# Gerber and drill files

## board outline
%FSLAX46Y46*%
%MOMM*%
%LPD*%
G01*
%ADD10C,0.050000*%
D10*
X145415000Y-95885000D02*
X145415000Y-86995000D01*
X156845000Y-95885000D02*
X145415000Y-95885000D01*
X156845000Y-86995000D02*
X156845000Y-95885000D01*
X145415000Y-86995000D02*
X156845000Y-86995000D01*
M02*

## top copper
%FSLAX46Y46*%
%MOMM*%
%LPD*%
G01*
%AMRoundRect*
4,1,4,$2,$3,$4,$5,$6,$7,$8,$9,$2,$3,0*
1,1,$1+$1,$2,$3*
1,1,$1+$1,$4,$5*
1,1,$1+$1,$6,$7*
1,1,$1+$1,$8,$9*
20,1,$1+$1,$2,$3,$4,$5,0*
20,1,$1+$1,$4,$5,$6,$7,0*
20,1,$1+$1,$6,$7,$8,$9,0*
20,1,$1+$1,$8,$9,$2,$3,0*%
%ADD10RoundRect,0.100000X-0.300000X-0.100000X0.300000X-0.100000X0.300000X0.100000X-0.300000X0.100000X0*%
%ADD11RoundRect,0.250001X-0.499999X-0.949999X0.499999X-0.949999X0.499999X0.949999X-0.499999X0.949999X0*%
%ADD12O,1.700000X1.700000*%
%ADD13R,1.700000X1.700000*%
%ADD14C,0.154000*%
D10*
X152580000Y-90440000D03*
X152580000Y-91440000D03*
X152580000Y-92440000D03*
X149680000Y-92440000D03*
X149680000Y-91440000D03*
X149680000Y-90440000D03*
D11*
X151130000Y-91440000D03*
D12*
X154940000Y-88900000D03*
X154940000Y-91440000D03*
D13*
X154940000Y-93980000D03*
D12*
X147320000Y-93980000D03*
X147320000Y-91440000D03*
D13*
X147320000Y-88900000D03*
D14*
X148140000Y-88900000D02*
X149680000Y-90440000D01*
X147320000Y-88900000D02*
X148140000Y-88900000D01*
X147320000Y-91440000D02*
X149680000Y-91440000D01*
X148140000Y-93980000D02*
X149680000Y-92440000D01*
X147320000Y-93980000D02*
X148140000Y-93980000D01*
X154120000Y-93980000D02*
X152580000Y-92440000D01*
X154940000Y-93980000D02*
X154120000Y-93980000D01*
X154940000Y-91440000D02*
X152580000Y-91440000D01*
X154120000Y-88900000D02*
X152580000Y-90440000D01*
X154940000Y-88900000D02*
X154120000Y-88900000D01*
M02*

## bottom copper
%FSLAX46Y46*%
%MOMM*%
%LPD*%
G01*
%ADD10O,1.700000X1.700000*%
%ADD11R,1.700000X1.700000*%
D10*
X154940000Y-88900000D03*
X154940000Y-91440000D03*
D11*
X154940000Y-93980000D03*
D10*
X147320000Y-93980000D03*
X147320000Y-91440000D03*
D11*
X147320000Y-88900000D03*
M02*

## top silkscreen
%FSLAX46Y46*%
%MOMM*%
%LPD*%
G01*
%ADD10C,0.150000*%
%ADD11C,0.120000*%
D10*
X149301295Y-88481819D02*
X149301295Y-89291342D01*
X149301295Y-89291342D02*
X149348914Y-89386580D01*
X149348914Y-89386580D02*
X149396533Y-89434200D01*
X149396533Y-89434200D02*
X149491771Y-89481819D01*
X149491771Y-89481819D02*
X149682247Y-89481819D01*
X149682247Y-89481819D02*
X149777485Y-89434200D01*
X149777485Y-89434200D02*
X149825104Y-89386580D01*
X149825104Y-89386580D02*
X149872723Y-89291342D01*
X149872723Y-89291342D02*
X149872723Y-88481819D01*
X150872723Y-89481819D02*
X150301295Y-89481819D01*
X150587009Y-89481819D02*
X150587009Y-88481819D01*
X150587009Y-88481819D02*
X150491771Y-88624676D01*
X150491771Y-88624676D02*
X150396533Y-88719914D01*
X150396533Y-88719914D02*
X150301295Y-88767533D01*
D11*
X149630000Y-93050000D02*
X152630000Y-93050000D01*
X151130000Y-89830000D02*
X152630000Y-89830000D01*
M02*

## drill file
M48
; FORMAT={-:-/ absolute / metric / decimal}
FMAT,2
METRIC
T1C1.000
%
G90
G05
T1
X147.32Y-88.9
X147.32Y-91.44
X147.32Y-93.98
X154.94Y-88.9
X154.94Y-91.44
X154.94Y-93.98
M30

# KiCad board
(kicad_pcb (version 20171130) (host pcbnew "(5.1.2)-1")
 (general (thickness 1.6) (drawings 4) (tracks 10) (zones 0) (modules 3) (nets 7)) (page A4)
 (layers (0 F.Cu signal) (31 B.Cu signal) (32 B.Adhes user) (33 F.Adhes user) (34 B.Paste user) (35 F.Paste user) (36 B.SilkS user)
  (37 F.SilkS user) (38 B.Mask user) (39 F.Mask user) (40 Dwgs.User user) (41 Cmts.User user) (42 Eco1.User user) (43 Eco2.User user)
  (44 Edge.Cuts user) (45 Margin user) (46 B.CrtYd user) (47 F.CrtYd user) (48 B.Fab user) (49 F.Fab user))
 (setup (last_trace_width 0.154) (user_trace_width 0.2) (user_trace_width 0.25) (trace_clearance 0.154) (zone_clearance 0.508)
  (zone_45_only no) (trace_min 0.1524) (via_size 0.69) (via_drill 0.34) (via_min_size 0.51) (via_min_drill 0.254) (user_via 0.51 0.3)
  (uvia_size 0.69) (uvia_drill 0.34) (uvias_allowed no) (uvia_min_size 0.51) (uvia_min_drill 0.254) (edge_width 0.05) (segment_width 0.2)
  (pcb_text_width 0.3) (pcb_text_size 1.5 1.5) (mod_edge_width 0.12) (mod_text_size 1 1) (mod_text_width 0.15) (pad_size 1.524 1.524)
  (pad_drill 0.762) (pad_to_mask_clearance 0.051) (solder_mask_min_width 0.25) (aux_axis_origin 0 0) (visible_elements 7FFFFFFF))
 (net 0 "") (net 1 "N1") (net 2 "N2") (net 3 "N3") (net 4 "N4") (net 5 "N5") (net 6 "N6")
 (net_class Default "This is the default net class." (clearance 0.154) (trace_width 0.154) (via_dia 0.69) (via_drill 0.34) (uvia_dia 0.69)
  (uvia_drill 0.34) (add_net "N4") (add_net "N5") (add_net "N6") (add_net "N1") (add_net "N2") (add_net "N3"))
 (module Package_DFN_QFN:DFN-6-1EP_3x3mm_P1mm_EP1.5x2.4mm (layer F.Cu) (at 151.13 91.44)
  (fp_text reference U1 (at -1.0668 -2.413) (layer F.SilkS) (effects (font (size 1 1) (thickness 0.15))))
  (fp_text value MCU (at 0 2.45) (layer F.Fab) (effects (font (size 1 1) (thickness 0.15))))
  (fp_line (start -1.5 1.61) (end 1.5 1.61) (layer F.SilkS) (width 0.12))
  (fp_line (start 0 -1.61) (end 1.5 -1.61) (layer F.SilkS) (width 0.12))
  (pad 6 smd roundrect (at 1.45 -1) (size 0.8 0.4) (layers F.Cu F.Paste F.Mask) (roundrect_rratio 0.25) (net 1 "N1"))
  (pad 5 smd roundrect (at 1.45 0) (size 0.8 0.4) (layers F.Cu F.Paste F.Mask) (roundrect_rratio 0.25) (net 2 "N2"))
  (pad 4 smd roundrect (at 1.45 1) (size 0.8 0.4) (layers F.Cu F.Paste F.Mask) (roundrect_rratio 0.25) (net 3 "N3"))
  (pad 3 smd roundrect (at -1.45 1) (size 0.8 0.4) (layers F.Cu F.Paste F.Mask) (roundrect_rratio 0.25) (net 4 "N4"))
  (pad 2 smd roundrect (at -1.45 0) (size 0.8 0.4) (layers F.Cu F.Paste F.Mask) (roundrect_rratio 0.25) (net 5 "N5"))
  (pad 1 smd roundrect (at -1.45 -1) (size 0.8 0.4) (layers F.Cu F.Paste F.Mask) (roundrect_rratio 0.25) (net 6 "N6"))
  (pad "" smd roundrect (at 0.375 0.6) (size 0.6 0.97) (layers F.Paste) (roundrect_rratio 0.25))
  (pad "" smd roundrect (at 0.375 -0.6) (size 0.6 0.97) (layers F.Paste) (roundrect_rratio 0.25))
  (pad "" smd roundrect (at -0.375 0.6) (size 0.6 0.97) (layers F.Paste) (roundrect_rratio 0.25))
  (pad "" smd roundrect (at -0.375 -0.6) (size 0.6 0.97) (layers F.Paste) (roundrect_rratio 0.25))
  (pad 7 smd roundrect (at 0 0) (size 1.5 2.4) (layers F.Cu F.Mask) (roundrect_rratio 0.166667)))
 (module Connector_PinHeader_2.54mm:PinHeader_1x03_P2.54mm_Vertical (layer B.Cu) (at 154.94 93.98)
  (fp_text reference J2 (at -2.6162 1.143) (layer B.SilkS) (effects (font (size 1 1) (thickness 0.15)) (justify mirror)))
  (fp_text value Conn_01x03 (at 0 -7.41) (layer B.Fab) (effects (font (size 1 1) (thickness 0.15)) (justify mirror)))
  (pad 3 thru_hole oval (at 0 -5.08) (size 1.7 1.7) (drill 1) (layers *.Cu *.Mask) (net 3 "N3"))
  (pad 2 thru_hole oval (at 0 -2.54) (size 1.7 1.7) (drill 1) (layers *.Cu *.Mask) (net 2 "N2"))
  (pad 1 thru_hole rect (at 0 0) (size 1.7 1.7) (drill 1) (layers *.Cu *.Mask) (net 1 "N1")))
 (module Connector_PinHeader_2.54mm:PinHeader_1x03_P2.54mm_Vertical (layer B.Cu) (at 147.32 88.9 180)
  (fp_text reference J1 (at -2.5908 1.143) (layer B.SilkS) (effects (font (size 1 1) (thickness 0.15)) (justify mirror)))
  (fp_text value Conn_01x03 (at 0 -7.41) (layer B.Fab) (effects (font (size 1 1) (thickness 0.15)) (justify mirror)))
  (pad 3 thru_hole oval (at 0 -5.08 180) (size 1.7 1.7) (drill 1) (layers *.Cu *.Mask) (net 6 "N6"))
  (pad 2 thru_hole oval (at 0 -2.54 180) (size 1.7 1.7) (drill 1) (layers *.Cu *.Mask) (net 5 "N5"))
  (pad 1 thru_hole rect (at 0 0 180) (size 1.7 1.7) (drill 1) (layers *.Cu *.Mask) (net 4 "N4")))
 (gr_line (start 145.415 95.885) (end 145.415 86.995) (layer Edge.Cuts) (width 0.05))
 (gr_line (start 156.845 95.885) (end 145.415 95.885) (layer Edge.Cuts) (width 0.05))
 (gr_line (start 156.845 86.995) (end 156.845 95.885) (layer Edge.Cuts) (width 0.05))
 (gr_line (start 145.415 86.995) (end 156.845 86.995) (layer Edge.Cuts) (width 0.05))
 (segment (start 148.14 88.9) (end 149.68 90.44) (width 0.154) (layer F.Cu) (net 6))
 (segment (start 147.32 88.9) (end 148.14 88.9) (width 0.154) (layer F.Cu) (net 6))
 (segment (start 147.32 91.44) (end 149.68 91.44) (width 0.154) (layer F.Cu) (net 5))
 (segment (start 148.14 93.98) (end 149.68 92.44) (width 0.154) (layer F.Cu) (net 4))
 (segment (start 147.32 93.98) (end 148.14 93.98) (width 0.154) (layer F.Cu) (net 4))
 (segment (start 154.12 93.98) (end 152.58 92.44) (width 0.154) (layer F.Cu) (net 3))
 (segment (start 154.94 93.98) (end 154.12 93.98) (width 0.154) (layer F.Cu) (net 3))
 (segment (start 154.94 91.44) (end 152.58 91.44) (width 0.154) (layer F.Cu) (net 2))
 (segment (start 154.12 88.9) (end 152.58 90.44) (width 0.154) (layer F.Cu) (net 1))
 (segment (start 154.94 88.9) (end 154.12 88.9) (width 0.154) (layer F.Cu) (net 1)))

